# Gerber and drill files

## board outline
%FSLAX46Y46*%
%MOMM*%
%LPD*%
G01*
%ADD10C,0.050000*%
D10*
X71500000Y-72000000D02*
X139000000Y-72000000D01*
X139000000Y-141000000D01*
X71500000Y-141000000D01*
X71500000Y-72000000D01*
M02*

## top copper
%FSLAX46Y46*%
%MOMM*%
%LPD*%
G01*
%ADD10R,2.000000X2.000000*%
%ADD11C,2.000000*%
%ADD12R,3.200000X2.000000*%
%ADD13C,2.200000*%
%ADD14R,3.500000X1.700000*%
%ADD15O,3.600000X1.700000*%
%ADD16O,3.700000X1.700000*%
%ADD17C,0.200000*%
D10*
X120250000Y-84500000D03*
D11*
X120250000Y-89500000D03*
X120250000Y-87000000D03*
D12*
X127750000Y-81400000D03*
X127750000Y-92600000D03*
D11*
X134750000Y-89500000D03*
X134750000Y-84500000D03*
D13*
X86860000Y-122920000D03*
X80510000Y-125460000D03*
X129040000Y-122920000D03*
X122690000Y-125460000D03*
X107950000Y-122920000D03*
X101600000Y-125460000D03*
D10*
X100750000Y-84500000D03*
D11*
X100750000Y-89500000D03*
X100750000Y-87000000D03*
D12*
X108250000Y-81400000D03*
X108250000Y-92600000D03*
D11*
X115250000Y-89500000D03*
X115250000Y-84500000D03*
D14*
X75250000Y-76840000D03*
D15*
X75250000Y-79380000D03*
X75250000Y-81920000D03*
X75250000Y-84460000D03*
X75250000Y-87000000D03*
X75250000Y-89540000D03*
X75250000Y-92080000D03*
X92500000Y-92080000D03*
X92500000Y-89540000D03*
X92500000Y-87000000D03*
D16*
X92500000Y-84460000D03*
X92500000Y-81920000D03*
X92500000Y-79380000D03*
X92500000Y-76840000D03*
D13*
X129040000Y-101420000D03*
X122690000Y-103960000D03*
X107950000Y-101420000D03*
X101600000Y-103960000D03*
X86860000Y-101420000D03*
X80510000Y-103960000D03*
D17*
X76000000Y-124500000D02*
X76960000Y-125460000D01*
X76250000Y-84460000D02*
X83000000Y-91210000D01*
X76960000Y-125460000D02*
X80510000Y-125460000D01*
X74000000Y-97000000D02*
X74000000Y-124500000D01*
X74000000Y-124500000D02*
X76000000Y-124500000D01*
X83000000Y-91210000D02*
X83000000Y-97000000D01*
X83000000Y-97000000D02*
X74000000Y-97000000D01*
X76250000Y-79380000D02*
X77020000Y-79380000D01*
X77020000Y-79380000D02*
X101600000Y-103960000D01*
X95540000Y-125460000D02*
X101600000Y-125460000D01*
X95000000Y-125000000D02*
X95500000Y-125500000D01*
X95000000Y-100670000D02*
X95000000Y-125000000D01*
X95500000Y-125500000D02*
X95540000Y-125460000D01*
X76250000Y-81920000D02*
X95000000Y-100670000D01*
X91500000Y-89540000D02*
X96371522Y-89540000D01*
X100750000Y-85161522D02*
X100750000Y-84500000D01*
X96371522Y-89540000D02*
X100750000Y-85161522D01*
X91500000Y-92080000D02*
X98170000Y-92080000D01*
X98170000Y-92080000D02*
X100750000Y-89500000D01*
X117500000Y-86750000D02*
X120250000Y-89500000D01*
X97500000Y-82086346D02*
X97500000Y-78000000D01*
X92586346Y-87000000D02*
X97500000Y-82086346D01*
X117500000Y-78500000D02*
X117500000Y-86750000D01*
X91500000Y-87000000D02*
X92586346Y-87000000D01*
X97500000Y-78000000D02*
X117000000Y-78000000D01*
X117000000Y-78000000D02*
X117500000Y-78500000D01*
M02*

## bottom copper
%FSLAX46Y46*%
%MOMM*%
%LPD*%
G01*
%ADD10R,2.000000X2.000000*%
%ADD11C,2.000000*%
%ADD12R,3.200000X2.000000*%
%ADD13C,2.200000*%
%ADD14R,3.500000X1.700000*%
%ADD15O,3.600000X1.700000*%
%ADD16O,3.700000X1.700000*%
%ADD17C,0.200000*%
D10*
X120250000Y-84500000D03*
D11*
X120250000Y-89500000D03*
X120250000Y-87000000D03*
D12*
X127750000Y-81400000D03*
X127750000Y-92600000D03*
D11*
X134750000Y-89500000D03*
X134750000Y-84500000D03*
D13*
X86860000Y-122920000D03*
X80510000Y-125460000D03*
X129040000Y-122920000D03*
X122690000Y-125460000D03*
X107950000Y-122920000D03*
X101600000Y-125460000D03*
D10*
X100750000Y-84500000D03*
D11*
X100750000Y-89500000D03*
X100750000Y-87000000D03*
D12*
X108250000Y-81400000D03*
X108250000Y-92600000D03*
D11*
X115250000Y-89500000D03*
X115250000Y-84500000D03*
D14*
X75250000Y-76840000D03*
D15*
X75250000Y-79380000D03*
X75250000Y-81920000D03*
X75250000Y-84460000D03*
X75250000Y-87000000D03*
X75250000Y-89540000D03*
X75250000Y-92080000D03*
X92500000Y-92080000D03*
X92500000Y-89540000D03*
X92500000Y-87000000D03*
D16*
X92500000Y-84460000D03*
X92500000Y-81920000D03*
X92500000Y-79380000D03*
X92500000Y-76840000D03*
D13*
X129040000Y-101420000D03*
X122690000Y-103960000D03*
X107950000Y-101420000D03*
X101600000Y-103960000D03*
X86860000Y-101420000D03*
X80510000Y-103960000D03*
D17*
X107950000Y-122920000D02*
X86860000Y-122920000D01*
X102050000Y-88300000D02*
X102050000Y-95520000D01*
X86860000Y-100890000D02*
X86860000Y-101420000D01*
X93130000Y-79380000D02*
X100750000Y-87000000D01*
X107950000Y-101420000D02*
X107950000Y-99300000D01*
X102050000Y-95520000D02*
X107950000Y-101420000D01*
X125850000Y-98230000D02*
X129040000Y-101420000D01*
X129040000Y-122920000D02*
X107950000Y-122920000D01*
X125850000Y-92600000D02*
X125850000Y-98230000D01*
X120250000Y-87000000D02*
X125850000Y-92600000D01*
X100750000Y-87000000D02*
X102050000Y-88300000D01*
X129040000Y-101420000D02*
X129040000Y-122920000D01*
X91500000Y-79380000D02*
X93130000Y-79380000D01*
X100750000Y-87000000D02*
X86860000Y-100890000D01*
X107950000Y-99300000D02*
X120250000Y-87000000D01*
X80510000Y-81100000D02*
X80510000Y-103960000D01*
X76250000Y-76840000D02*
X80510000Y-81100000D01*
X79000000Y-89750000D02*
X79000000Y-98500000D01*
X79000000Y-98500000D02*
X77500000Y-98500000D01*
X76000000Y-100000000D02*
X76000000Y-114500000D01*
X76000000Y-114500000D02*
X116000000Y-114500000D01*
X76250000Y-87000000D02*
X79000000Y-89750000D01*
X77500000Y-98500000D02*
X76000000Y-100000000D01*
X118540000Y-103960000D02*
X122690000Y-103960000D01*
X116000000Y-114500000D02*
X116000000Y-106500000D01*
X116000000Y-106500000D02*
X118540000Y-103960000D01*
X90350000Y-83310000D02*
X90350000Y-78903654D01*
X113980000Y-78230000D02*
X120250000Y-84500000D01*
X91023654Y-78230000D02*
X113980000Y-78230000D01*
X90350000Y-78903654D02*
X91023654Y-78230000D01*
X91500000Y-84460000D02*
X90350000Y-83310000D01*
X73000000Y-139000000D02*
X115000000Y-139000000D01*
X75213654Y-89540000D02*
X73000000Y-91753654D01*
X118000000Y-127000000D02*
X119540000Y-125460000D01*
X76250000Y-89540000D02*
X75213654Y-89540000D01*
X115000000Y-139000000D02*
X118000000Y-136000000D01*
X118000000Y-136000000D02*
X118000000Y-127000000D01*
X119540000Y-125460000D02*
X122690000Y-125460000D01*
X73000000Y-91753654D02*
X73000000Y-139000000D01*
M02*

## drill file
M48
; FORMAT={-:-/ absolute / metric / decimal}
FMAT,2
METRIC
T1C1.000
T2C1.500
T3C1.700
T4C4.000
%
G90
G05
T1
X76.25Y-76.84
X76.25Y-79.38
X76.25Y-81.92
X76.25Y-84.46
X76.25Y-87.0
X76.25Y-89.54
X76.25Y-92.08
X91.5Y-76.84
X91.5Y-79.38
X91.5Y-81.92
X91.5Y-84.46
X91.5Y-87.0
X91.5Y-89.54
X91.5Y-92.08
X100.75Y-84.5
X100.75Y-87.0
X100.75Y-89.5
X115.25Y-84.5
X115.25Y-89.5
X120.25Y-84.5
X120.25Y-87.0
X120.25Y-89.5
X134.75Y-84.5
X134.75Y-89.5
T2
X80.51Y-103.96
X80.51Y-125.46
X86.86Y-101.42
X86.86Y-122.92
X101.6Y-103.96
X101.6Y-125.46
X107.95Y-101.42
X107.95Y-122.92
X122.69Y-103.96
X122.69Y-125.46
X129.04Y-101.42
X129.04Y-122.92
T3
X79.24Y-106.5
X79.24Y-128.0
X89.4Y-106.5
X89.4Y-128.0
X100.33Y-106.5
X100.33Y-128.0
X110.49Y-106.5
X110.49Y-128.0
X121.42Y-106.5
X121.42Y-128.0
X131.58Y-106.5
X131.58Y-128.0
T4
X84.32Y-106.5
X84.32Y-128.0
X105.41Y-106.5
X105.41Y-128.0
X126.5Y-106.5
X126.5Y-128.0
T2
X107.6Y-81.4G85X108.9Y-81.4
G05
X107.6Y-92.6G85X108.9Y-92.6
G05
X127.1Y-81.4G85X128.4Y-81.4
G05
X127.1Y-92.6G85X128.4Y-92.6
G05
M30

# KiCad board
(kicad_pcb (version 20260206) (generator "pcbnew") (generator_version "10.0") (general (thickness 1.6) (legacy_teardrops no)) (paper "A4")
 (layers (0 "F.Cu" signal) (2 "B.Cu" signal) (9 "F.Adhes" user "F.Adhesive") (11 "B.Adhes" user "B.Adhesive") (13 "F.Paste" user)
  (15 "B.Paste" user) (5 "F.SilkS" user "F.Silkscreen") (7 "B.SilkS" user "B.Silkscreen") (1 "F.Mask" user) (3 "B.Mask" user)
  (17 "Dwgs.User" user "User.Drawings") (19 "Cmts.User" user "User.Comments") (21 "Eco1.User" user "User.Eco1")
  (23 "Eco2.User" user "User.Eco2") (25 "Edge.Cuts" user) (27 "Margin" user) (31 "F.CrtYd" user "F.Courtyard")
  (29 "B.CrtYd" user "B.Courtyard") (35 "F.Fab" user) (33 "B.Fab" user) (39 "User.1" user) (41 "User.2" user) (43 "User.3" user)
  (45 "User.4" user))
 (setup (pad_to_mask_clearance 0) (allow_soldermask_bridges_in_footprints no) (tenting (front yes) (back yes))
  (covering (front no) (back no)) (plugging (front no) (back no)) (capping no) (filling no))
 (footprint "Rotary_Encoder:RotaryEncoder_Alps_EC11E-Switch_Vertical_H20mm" (layer "F.Cu") (at 120.25 84.5)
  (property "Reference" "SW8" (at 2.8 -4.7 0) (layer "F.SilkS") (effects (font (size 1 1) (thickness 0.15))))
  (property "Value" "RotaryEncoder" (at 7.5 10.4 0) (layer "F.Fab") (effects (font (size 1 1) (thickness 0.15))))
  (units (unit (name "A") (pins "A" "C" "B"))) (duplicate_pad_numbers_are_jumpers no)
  (pad "A" thru_hole rect (at 0 0) (size 2 2) (drill 1) (layers "*.Cu" "*.Mask") (remove_unused_layers no) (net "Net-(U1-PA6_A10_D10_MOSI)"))
  (pad "B" thru_hole circle (at 0 5) (size 2 2) (drill 1) (layers "*.Cu" "*.Mask") (remove_unused_layers no) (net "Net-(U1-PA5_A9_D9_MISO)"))
  (pad "C" thru_hole circle (at 0 2.5) (size 2 2) (drill 1) (layers "*.Cu" "*.Mask") (remove_unused_layers no) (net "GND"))
  (pad "MP" thru_hole rect (at 7.5 -3.1) (size 3.2 2) (drill oval 2.8 1.5) (layers "*.Cu" "*.Mask") (remove_unused_layers no))
  (pad "MP" thru_hole rect (at 7.5 8.1) (size 3.2 2) (drill oval 2.8 1.5) (layers "*.Cu" "*.Mask") (remove_unused_layers no))
  (pad "S1" thru_hole circle (at 14.5 5) (size 2 2) (drill 1) (layers "*.Cu" "*.Mask") (remove_unused_layers no))
  (pad "S2" thru_hole circle (at 14.5 0) (size 2 2) (drill 1) (layers "*.Cu" "*.Mask") (remove_unused_layers no)))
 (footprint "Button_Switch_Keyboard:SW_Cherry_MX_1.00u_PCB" (layer "F.Cu") (at 86.86 122.92)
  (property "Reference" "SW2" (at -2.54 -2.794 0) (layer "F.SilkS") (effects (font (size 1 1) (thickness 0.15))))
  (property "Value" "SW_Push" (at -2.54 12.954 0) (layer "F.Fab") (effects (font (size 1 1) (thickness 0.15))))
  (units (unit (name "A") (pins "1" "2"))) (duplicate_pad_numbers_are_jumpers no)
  (pad "" np_thru_hole circle (at -7.62 5.08) (size 1.7 1.7) (drill 1.7) (layers "*.Cu" "*.Mask"))
  (pad "" np_thru_hole circle (at -2.54 5.08) (size 4 4) (drill 4) (layers "*.Cu" "*.Mask"))
  (pad "" np_thru_hole circle (at 2.54 5.08) (size 1.7 1.7) (drill 1.7) (layers "*.Cu" "*.Mask"))
  (pad "1" thru_hole circle (at 0 0) (size 2.2 2.2) (drill 1.5) (layers "*.Cu" "*.Mask") (remove_unused_layers no) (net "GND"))
  (pad "2" thru_hole circle (at -6.35 2.54) (size 2.2 2.2) (drill 1.5) (layers "*.Cu" "*.Mask") (remove_unused_layers no)
   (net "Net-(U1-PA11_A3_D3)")))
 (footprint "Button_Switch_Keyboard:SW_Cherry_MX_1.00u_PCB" (layer "F.Cu") (at 129.04 122.92)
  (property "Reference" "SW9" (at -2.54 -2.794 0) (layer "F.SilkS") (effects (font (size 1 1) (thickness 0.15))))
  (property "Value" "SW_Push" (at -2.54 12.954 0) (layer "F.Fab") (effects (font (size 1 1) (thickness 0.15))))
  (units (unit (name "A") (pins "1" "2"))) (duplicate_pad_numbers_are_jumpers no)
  (pad "" np_thru_hole circle (at -7.62 5.08) (size 1.7 1.7) (drill 1.7) (layers "*.Cu" "*.Mask"))
  (pad "" np_thru_hole circle (at -2.54 5.08) (size 4 4) (drill 4) (layers "*.Cu" "*.Mask"))
  (pad "" np_thru_hole circle (at 2.54 5.08) (size 1.7 1.7) (drill 1.7) (layers "*.Cu" "*.Mask"))
  (pad "1" thru_hole circle (at 0 0) (size 2.2 2.2) (drill 1.5) (layers "*.Cu" "*.Mask") (remove_unused_layers no) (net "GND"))
  (pad "2" thru_hole circle (at -6.35 2.54) (size 2.2 2.2) (drill 1.5) (layers "*.Cu" "*.Mask") (remove_unused_layers no)
   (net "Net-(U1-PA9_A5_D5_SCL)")))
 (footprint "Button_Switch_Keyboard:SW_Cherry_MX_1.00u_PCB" (layer "F.Cu") (at 107.95 122.92)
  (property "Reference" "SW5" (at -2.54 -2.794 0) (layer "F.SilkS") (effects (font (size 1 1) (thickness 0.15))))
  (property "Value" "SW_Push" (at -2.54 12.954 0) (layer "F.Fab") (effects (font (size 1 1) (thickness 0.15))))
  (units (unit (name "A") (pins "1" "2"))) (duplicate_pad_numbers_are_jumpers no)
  (pad "" np_thru_hole circle (at -7.62 5.08) (size 1.7 1.7) (drill 1.7) (layers "*.Cu" "*.Mask"))
  (pad "" np_thru_hole circle (at -2.54 5.08) (size 4 4) (drill 4) (layers "*.Cu" "*.Mask"))
  (pad "" np_thru_hole circle (at 2.54 5.08) (size 1.7 1.7) (drill 1.7) (layers "*.Cu" "*.Mask"))
  (pad "1" thru_hole circle (at 0 0) (size 2.2 2.2) (drill 1.5) (layers "*.Cu" "*.Mask") (remove_unused_layers no) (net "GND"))
  (pad "2" thru_hole circle (at -6.35 2.54) (size 2.2 2.2) (drill 1.5) (layers "*.Cu" "*.Mask") (remove_unused_layers no)
   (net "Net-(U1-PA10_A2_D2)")))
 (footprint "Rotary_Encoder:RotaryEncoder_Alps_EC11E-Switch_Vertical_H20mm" (layer "F.Cu") (at 100.75 84.5)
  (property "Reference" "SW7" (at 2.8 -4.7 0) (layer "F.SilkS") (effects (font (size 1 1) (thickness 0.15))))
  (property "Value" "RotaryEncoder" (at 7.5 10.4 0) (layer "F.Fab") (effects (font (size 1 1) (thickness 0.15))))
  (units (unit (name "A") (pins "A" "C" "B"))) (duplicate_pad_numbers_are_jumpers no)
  (pad "A" thru_hole rect (at 0 0) (size 2 2) (drill 1) (layers "*.Cu" "*.Mask") (remove_unused_layers no) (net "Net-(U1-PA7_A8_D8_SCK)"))
  (pad "B" thru_hole circle (at 0 5) (size 2 2) (drill 1) (layers "*.Cu" "*.Mask") (remove_unused_layers no) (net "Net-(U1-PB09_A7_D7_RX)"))
  (pad "C" thru_hole circle (at 0 2.5) (size 2 2) (drill 1) (layers "*.Cu" "*.Mask") (remove_unused_layers no) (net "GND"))
  (pad "MP" thru_hole rect (at 7.5 -3.1) (size 3.2 2) (drill oval 2.8 1.5) (layers "*.Cu" "*.Mask") (remove_unused_layers no))
  (pad "MP" thru_hole rect (at 7.5 8.1) (size 3.2 2) (drill oval 2.8 1.5) (layers "*.Cu" "*.Mask") (remove_unused_layers no))
  (pad "S1" thru_hole circle (at 14.5 5) (size 2 2) (drill 1) (layers "*.Cu" "*.Mask") (remove_unused_layers no))
  (pad "S2" thru_hole circle (at 14.5 0) (size 2 2) (drill 1) (layers "*.Cu" "*.Mask") (remove_unused_layers no)))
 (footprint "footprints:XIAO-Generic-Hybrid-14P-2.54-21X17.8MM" (layer "F.Cu") (at 83.875 84.46)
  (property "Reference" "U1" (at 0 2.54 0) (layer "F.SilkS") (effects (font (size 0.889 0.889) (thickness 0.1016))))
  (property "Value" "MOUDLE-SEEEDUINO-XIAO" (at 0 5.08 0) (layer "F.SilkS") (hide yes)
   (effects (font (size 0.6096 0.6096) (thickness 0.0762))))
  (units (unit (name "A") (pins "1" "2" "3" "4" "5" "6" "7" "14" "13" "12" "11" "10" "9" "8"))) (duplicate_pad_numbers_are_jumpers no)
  (pad "1" thru_hole rect (at -7.625 -7.62) (size 3.5 1.7) (drill 1 (offset -1 0)) (layers "*.Cu" "*.Mask") (remove_unused_layers no)
   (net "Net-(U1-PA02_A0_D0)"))
  (pad "2" thru_hole oval (at -7.625 -5.08) (size 3.6 1.7) (drill 1 (offset -1 0)) (layers "*.Cu" "*.Mask") (remove_unused_layers no)
   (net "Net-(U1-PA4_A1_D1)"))
  (pad "3" thru_hole oval (at -7.625 -2.54) (size 3.6 1.7) (drill 1 (offset -1 0)) (layers "*.Cu" "*.Mask") (remove_unused_layers no)
   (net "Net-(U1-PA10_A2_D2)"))
  (pad "4" thru_hole oval (at -7.625 0) (size 3.6 1.7) (drill 1 (offset -1 0)) (layers "*.Cu" "*.Mask") (remove_unused_layers no)
   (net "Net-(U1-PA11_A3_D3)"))
  (pad "5" thru_hole oval (at -7.625 2.54) (size 3.6 1.7) (drill 1 (offset -1 0)) (layers "*.Cu" "*.Mask") (remove_unused_layers no)
   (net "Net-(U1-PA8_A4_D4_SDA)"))
  (pad "6" thru_hole oval (at -7.625 5.08 180) (size 3.6 1.7) (drill 1 (offset 1 0)) (layers "*.Cu" "*.Mask") (remove_unused_layers no)
   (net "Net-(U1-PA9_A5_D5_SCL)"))
  (pad "7" thru_hole oval (at -7.625 7.62) (size 3.6 1.7) (drill 1 (offset -1 0)) (layers "*.Cu" "*.Mask") (remove_unused_layers no)
   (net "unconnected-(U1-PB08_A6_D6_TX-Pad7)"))
  (pad "8" thru_hole oval (at 7.625 7.62) (size 3.6 1.7) (drill 1 (offset 1 0)) (layers "*.Cu" "*.Mask") (remove_unused_layers no)
   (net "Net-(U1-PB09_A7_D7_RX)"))
  (pad "9" thru_hole oval (at 7.625 5.08) (size 3.6 1.7) (drill 1 (offset 1 0)) (layers "*.Cu" "*.Mask") (remove_unused_layers no)
   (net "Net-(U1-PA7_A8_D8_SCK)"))
  (pad "10" thru_hole oval (at 7.625 2.54) (size 3.6 1.7) (drill 1 (offset 1 0)) (layers "*.Cu" "*.Mask") (remove_unused_layers no)
   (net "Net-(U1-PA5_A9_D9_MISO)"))
  (pad "11" thru_hole oval (at 7.625 0) (size 3.7 1.7) (drill 1 (offset 1 0)) (layers "*.Cu" "*.Mask") (remove_unused_layers no)
   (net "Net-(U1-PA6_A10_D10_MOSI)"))
  (pad "12" thru_hole oval (at 7.625 -2.54) (size 3.7 1.7) (drill 1 (offset 1 0)) (layers "*.Cu" "*.Mask") (remove_unused_layers no)
   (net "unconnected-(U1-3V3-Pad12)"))
  (pad "13" thru_hole oval (at 7.625 -5.08) (size 3.7 1.7) (drill 1 (offset 1 0)) (layers "*.Cu" "*.Mask") (remove_unused_layers no)
   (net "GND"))
  (pad "14" thru_hole oval (at 7.625 -7.62) (size 3.7 1.7) (drill 1 (offset 1 0)) (layers "*.Cu" "*.Mask") (remove_unused_layers no)
   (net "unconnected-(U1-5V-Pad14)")))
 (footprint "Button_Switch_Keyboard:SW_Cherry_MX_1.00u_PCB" (layer "F.Cu") (at 129.04 101.42)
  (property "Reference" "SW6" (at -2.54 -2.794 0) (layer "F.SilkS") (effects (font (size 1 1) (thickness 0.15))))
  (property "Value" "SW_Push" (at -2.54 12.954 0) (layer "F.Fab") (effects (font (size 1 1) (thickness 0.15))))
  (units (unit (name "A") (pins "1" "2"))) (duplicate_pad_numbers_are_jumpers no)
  (pad "" np_thru_hole circle (at -7.62 5.08) (size 1.7 1.7) (drill 1.7) (layers "*.Cu" "*.Mask"))
  (pad "" np_thru_hole circle (at -2.54 5.08) (size 4 4) (drill 4) (layers "*.Cu" "*.Mask"))
  (pad "" np_thru_hole circle (at 2.54 5.08) (size 1.7 1.7) (drill 1.7) (layers "*.Cu" "*.Mask"))
  (pad "1" thru_hole circle (at 0 0) (size 2.2 2.2) (drill 1.5) (layers "*.Cu" "*.Mask") (remove_unused_layers no) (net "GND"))
  (pad "2" thru_hole circle (at -6.35 2.54) (size 2.2 2.2) (drill 1.5) (layers "*.Cu" "*.Mask") (remove_unused_layers no)
   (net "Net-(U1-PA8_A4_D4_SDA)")))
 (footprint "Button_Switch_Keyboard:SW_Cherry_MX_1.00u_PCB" (layer "F.Cu") (at 107.95 101.42)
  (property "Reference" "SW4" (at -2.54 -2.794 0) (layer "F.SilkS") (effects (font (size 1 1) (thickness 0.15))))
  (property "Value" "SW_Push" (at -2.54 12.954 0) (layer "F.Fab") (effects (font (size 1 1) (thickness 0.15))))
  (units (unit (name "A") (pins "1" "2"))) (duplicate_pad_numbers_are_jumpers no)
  (pad "" np_thru_hole circle (at -7.62 5.08) (size 1.7 1.7) (drill 1.7) (layers "*.Cu" "*.Mask"))
  (pad "" np_thru_hole circle (at -2.54 5.08) (size 4 4) (drill 4) (layers "*.Cu" "*.Mask"))
  (pad "" np_thru_hole circle (at 2.54 5.08) (size 1.7 1.7) (drill 1.7) (layers "*.Cu" "*.Mask"))
  (pad "1" thru_hole circle (at 0 0) (size 2.2 2.2) (drill 1.5) (layers "*.Cu" "*.Mask") (remove_unused_layers no) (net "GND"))
  (pad "2" thru_hole circle (at -6.35 2.54) (size 2.2 2.2) (drill 1.5) (layers "*.Cu" "*.Mask") (remove_unused_layers no)
   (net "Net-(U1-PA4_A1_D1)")))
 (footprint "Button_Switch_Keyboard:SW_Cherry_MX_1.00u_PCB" (layer "F.Cu") (at 86.86 101.42)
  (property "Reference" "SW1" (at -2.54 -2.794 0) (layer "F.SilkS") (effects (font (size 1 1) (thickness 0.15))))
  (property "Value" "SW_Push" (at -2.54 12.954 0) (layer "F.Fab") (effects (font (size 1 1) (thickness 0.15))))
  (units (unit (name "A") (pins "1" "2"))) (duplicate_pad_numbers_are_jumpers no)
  (pad "" np_thru_hole circle (at -7.62 5.08) (size 1.7 1.7) (drill 1.7) (layers "*.Cu" "*.Mask"))
  (pad "" np_thru_hole circle (at -2.54 5.08) (size 4 4) (drill 4) (layers "*.Cu" "*.Mask"))
  (pad "" np_thru_hole circle (at 2.54 5.08) (size 1.7 1.7) (drill 1.7) (layers "*.Cu" "*.Mask"))
  (pad "1" thru_hole circle (at 0 0) (size 2.2 2.2) (drill 1.5) (layers "*.Cu" "*.Mask") (remove_unused_layers no) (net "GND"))
  (pad "2" thru_hole circle (at -6.35 2.54) (size 2.2 2.2) (drill 1.5) (layers "*.Cu" "*.Mask") (remove_unused_layers no)
   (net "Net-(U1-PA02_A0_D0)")))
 (gr_rect (start 71.5 72) (end 139 141) (stroke (width 0.05) (type default)) (fill no) (layer "Edge.Cuts"))
 (segment (start 107.95 122.92) (end 86.86 122.92) (width 0.2) (layer "B.Cu") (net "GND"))
 (segment (start 102.05 88.3) (end 102.05 95.52) (width 0.2) (layer "B.Cu") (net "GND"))
 (segment (start 86.86 100.89) (end 86.86 101.42) (width 0.2) (layer "B.Cu") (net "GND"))
 (segment (start 93.13 79.38) (end 100.75 87) (width 0.2) (layer "B.Cu") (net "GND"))
 (segment (start 107.95 101.42) (end 107.95 99.3) (width 0.2) (layer "B.Cu") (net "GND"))
 (segment (start 102.05 95.52) (end 107.95 101.42) (width 0.2) (layer "B.Cu") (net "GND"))
 (segment (start 125.85 98.23) (end 129.04 101.42) (width 0.2) (layer "B.Cu") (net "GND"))
 (segment (start 129.04 122.92) (end 107.95 122.92) (width 0.2) (layer "B.Cu") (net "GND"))
 (segment (start 125.85 92.6) (end 125.85 98.23) (width 0.2) (layer "B.Cu") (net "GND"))
 (segment (start 120.25 87) (end 125.85 92.6) (width 0.2) (layer "B.Cu") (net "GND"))
 (segment (start 100.75 87) (end 102.05 88.3) (width 0.2) (layer "B.Cu") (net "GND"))
 (segment (start 129.04 101.42) (end 129.04 122.92) (width 0.2) (layer "B.Cu") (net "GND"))
 (segment (start 91.5 79.38) (end 93.13 79.38) (width 0.2) (layer "B.Cu") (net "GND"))
 (segment (start 100.75 87) (end 86.86 100.89) (width 0.2) (layer "B.Cu") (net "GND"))
 (segment (start 107.95 99.3) (end 120.25 87) (width 0.2) (layer "B.Cu") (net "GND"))
 (segment (start 80.51 81.1) (end 80.51 103.96) (width 0.2) (layer "B.Cu") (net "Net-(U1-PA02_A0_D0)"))
 (segment (start 76.25 76.84) (end 80.51 81.1) (width 0.2) (layer "B.Cu") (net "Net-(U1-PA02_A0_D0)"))
 (segment (start 76 124.5) (end 76.96 125.46) (width 0.2) (layer "F.Cu") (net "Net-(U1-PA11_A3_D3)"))
 (segment (start 76.25 84.46) (end 83 91.21) (width 0.2) (layer "F.Cu") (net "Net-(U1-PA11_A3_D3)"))
 (segment (start 76.96 125.46) (end 80.51 125.46) (width 0.2) (layer "F.Cu") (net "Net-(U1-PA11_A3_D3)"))
 (segment (start 74 97) (end 74 124.5) (width 0.2) (layer "F.Cu") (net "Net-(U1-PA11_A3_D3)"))
 (segment (start 74 124.5) (end 76 124.5) (width 0.2) (layer "F.Cu") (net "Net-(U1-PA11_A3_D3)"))
 (segment (start 83 91.21) (end 83 97) (width 0.2) (layer "F.Cu") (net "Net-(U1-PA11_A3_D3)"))
 (segment (start 83 97) (end 74 97) (width 0.2) (layer "F.Cu") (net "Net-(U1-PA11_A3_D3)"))
 (segment (start 76.25 79.38) (end 77.02 79.38) (width 0.2) (layer "F.Cu") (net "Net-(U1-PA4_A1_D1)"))
 (segment (start 77.02 79.38) (end 101.6 103.96) (width 0.2) (layer "F.Cu") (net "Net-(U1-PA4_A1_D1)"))
 (segment (start 95.54 125.46) (end 101.6 125.46) (width 0.2) (layer "F.Cu") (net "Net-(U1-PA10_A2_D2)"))
 (segment (start 95 125) (end 95.5 125.5) (width 0.2) (layer "F.Cu") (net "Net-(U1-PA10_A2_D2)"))
 (segment (start 95 100.67) (end 95 125) (width 0.2) (layer "F.Cu") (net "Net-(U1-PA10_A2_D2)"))
 (segment (start 95.5 125.5) (end 95.54 125.46) (width 0.2) (layer "F.Cu") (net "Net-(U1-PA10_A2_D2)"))
 (segment (start 76.25 81.92) (end 95 100.67) (width 0.2) (layer "F.Cu") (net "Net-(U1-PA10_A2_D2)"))
 (segment (start 79 89.75) (end 79 98.5) (width 0.2) (layer "B.Cu") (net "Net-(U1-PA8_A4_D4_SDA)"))
 (segment (start 79 98.5) (end 77.5 98.5) (width 0.2) (layer "B.Cu") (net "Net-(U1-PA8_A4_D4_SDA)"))
 (segment (start 76 100) (end 76 114.5) (width 0.2) (layer "B.Cu") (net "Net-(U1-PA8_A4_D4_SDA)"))
 (segment (start 76 114.5) (end 116 114.5) (width 0.2) (layer "B.Cu") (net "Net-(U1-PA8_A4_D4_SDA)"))
 (segment (start 76.25 87) (end 79 89.75) (width 0.2) (layer "B.Cu") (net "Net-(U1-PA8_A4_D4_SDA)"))
 (segment (start 77.5 98.5) (end 76 100) (width 0.2) (layer "B.Cu") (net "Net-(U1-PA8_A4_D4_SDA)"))
 (segment (start 118.54 103.96) (end 122.69 103.96) (width 0.2) (layer "B.Cu") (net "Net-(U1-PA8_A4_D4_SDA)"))
 (segment (start 116 114.5) (end 116 106.5) (width 0.2) (layer "B.Cu") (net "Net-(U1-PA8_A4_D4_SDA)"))
 (segment (start 116 106.5) (end 118.54 103.96) (width 0.2) (layer "B.Cu") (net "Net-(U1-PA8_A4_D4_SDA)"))
 (segment (start 91.5 89.54) (end 96.371522 89.54) (width 0.2) (layer "F.Cu") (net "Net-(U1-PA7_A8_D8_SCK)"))
 (segment (start 100.75 85.161522) (end 100.75 84.5) (width 0.2) (layer "F.Cu") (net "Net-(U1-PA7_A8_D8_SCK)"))
 (segment (start 96.371522 89.54) (end 100.75 85.161522) (width 0.2) (layer "F.Cu") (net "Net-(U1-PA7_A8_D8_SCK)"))
 (segment (start 91.5 92.08) (end 98.17 92.08) (width 0.2) (layer "F.Cu") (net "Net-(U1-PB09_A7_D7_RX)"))
 (segment (start 98.17 92.08) (end 100.75 89.5) (width 0.2) (layer "F.Cu") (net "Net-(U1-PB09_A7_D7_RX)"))
 (segment (start 117.5 86.75) (end 120.25 89.5) (width 0.2) (layer "F.Cu") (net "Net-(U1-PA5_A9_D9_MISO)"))
 (segment (start 97.5 82.086346) (end 97.5 78) (width 0.2) (layer "F.Cu") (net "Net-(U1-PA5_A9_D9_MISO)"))
 (segment (start 92.586346 87) (end 97.5 82.086346) (width 0.2) (layer "F.Cu") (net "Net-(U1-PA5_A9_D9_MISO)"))
 (segment (start 117.5 78.5) (end 117.5 86.75) (width 0.2) (layer "F.Cu") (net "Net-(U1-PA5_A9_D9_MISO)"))
 (segment (start 91.5 87) (end 92.586346 87) (width 0.2) (layer "F.Cu") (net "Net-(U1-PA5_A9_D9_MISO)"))
 (segment (start 97.5 78) (end 117 78) (width 0.2) (layer "F.Cu") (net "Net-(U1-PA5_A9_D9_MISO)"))
 (segment (start 117 78) (end 117.5 78.5) (width 0.2) (layer "F.Cu") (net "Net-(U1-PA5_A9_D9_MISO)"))
 (segment (start 90.35 83.31) (end 90.35 78.903654) (width 0.2) (layer "B.Cu") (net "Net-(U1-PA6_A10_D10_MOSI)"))
 (segment (start 113.98 78.23) (end 120.25 84.5) (width 0.2) (layer "B.Cu") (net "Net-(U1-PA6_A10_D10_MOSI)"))
 (segment (start 91.023654 78.23) (end 113.98 78.23) (width 0.2) (layer "B.Cu") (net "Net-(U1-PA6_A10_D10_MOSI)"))
 (segment (start 90.35 78.903654) (end 91.023654 78.23) (width 0.2) (layer "B.Cu") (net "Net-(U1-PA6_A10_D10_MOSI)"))
 (segment (start 91.5 84.46) (end 90.35 83.31) (width 0.2) (layer "B.Cu") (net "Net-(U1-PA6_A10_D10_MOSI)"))
 (segment (start 73 139) (end 115 139) (width 0.2) (layer "B.Cu") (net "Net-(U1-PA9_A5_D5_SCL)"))
 (segment (start 75.213654 89.54) (end 73 91.753654) (width 0.2) (layer "B.Cu") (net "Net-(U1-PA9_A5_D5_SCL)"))
 (segment (start 118 127) (end 119.54 125.46) (width 0.2) (layer "B.Cu") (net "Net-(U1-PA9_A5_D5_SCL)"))
 (segment (start 76.25 89.54) (end 75.213654 89.54) (width 0.2) (layer "B.Cu") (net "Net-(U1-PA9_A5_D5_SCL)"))
 (segment (start 115 139) (end 118 136) (width 0.2) (layer "B.Cu") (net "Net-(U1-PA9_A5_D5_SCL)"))
 (segment (start 118 136) (end 118 127) (width 0.2) (layer "B.Cu") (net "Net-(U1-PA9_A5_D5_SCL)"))
 (segment (start 119.54 125.46) (end 122.69 125.46) (width 0.2) (layer "B.Cu") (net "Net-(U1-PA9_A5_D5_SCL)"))
 (segment (start 73 91.753654) (end 73 139) (width 0.2) (layer "B.Cu") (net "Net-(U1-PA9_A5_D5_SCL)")))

